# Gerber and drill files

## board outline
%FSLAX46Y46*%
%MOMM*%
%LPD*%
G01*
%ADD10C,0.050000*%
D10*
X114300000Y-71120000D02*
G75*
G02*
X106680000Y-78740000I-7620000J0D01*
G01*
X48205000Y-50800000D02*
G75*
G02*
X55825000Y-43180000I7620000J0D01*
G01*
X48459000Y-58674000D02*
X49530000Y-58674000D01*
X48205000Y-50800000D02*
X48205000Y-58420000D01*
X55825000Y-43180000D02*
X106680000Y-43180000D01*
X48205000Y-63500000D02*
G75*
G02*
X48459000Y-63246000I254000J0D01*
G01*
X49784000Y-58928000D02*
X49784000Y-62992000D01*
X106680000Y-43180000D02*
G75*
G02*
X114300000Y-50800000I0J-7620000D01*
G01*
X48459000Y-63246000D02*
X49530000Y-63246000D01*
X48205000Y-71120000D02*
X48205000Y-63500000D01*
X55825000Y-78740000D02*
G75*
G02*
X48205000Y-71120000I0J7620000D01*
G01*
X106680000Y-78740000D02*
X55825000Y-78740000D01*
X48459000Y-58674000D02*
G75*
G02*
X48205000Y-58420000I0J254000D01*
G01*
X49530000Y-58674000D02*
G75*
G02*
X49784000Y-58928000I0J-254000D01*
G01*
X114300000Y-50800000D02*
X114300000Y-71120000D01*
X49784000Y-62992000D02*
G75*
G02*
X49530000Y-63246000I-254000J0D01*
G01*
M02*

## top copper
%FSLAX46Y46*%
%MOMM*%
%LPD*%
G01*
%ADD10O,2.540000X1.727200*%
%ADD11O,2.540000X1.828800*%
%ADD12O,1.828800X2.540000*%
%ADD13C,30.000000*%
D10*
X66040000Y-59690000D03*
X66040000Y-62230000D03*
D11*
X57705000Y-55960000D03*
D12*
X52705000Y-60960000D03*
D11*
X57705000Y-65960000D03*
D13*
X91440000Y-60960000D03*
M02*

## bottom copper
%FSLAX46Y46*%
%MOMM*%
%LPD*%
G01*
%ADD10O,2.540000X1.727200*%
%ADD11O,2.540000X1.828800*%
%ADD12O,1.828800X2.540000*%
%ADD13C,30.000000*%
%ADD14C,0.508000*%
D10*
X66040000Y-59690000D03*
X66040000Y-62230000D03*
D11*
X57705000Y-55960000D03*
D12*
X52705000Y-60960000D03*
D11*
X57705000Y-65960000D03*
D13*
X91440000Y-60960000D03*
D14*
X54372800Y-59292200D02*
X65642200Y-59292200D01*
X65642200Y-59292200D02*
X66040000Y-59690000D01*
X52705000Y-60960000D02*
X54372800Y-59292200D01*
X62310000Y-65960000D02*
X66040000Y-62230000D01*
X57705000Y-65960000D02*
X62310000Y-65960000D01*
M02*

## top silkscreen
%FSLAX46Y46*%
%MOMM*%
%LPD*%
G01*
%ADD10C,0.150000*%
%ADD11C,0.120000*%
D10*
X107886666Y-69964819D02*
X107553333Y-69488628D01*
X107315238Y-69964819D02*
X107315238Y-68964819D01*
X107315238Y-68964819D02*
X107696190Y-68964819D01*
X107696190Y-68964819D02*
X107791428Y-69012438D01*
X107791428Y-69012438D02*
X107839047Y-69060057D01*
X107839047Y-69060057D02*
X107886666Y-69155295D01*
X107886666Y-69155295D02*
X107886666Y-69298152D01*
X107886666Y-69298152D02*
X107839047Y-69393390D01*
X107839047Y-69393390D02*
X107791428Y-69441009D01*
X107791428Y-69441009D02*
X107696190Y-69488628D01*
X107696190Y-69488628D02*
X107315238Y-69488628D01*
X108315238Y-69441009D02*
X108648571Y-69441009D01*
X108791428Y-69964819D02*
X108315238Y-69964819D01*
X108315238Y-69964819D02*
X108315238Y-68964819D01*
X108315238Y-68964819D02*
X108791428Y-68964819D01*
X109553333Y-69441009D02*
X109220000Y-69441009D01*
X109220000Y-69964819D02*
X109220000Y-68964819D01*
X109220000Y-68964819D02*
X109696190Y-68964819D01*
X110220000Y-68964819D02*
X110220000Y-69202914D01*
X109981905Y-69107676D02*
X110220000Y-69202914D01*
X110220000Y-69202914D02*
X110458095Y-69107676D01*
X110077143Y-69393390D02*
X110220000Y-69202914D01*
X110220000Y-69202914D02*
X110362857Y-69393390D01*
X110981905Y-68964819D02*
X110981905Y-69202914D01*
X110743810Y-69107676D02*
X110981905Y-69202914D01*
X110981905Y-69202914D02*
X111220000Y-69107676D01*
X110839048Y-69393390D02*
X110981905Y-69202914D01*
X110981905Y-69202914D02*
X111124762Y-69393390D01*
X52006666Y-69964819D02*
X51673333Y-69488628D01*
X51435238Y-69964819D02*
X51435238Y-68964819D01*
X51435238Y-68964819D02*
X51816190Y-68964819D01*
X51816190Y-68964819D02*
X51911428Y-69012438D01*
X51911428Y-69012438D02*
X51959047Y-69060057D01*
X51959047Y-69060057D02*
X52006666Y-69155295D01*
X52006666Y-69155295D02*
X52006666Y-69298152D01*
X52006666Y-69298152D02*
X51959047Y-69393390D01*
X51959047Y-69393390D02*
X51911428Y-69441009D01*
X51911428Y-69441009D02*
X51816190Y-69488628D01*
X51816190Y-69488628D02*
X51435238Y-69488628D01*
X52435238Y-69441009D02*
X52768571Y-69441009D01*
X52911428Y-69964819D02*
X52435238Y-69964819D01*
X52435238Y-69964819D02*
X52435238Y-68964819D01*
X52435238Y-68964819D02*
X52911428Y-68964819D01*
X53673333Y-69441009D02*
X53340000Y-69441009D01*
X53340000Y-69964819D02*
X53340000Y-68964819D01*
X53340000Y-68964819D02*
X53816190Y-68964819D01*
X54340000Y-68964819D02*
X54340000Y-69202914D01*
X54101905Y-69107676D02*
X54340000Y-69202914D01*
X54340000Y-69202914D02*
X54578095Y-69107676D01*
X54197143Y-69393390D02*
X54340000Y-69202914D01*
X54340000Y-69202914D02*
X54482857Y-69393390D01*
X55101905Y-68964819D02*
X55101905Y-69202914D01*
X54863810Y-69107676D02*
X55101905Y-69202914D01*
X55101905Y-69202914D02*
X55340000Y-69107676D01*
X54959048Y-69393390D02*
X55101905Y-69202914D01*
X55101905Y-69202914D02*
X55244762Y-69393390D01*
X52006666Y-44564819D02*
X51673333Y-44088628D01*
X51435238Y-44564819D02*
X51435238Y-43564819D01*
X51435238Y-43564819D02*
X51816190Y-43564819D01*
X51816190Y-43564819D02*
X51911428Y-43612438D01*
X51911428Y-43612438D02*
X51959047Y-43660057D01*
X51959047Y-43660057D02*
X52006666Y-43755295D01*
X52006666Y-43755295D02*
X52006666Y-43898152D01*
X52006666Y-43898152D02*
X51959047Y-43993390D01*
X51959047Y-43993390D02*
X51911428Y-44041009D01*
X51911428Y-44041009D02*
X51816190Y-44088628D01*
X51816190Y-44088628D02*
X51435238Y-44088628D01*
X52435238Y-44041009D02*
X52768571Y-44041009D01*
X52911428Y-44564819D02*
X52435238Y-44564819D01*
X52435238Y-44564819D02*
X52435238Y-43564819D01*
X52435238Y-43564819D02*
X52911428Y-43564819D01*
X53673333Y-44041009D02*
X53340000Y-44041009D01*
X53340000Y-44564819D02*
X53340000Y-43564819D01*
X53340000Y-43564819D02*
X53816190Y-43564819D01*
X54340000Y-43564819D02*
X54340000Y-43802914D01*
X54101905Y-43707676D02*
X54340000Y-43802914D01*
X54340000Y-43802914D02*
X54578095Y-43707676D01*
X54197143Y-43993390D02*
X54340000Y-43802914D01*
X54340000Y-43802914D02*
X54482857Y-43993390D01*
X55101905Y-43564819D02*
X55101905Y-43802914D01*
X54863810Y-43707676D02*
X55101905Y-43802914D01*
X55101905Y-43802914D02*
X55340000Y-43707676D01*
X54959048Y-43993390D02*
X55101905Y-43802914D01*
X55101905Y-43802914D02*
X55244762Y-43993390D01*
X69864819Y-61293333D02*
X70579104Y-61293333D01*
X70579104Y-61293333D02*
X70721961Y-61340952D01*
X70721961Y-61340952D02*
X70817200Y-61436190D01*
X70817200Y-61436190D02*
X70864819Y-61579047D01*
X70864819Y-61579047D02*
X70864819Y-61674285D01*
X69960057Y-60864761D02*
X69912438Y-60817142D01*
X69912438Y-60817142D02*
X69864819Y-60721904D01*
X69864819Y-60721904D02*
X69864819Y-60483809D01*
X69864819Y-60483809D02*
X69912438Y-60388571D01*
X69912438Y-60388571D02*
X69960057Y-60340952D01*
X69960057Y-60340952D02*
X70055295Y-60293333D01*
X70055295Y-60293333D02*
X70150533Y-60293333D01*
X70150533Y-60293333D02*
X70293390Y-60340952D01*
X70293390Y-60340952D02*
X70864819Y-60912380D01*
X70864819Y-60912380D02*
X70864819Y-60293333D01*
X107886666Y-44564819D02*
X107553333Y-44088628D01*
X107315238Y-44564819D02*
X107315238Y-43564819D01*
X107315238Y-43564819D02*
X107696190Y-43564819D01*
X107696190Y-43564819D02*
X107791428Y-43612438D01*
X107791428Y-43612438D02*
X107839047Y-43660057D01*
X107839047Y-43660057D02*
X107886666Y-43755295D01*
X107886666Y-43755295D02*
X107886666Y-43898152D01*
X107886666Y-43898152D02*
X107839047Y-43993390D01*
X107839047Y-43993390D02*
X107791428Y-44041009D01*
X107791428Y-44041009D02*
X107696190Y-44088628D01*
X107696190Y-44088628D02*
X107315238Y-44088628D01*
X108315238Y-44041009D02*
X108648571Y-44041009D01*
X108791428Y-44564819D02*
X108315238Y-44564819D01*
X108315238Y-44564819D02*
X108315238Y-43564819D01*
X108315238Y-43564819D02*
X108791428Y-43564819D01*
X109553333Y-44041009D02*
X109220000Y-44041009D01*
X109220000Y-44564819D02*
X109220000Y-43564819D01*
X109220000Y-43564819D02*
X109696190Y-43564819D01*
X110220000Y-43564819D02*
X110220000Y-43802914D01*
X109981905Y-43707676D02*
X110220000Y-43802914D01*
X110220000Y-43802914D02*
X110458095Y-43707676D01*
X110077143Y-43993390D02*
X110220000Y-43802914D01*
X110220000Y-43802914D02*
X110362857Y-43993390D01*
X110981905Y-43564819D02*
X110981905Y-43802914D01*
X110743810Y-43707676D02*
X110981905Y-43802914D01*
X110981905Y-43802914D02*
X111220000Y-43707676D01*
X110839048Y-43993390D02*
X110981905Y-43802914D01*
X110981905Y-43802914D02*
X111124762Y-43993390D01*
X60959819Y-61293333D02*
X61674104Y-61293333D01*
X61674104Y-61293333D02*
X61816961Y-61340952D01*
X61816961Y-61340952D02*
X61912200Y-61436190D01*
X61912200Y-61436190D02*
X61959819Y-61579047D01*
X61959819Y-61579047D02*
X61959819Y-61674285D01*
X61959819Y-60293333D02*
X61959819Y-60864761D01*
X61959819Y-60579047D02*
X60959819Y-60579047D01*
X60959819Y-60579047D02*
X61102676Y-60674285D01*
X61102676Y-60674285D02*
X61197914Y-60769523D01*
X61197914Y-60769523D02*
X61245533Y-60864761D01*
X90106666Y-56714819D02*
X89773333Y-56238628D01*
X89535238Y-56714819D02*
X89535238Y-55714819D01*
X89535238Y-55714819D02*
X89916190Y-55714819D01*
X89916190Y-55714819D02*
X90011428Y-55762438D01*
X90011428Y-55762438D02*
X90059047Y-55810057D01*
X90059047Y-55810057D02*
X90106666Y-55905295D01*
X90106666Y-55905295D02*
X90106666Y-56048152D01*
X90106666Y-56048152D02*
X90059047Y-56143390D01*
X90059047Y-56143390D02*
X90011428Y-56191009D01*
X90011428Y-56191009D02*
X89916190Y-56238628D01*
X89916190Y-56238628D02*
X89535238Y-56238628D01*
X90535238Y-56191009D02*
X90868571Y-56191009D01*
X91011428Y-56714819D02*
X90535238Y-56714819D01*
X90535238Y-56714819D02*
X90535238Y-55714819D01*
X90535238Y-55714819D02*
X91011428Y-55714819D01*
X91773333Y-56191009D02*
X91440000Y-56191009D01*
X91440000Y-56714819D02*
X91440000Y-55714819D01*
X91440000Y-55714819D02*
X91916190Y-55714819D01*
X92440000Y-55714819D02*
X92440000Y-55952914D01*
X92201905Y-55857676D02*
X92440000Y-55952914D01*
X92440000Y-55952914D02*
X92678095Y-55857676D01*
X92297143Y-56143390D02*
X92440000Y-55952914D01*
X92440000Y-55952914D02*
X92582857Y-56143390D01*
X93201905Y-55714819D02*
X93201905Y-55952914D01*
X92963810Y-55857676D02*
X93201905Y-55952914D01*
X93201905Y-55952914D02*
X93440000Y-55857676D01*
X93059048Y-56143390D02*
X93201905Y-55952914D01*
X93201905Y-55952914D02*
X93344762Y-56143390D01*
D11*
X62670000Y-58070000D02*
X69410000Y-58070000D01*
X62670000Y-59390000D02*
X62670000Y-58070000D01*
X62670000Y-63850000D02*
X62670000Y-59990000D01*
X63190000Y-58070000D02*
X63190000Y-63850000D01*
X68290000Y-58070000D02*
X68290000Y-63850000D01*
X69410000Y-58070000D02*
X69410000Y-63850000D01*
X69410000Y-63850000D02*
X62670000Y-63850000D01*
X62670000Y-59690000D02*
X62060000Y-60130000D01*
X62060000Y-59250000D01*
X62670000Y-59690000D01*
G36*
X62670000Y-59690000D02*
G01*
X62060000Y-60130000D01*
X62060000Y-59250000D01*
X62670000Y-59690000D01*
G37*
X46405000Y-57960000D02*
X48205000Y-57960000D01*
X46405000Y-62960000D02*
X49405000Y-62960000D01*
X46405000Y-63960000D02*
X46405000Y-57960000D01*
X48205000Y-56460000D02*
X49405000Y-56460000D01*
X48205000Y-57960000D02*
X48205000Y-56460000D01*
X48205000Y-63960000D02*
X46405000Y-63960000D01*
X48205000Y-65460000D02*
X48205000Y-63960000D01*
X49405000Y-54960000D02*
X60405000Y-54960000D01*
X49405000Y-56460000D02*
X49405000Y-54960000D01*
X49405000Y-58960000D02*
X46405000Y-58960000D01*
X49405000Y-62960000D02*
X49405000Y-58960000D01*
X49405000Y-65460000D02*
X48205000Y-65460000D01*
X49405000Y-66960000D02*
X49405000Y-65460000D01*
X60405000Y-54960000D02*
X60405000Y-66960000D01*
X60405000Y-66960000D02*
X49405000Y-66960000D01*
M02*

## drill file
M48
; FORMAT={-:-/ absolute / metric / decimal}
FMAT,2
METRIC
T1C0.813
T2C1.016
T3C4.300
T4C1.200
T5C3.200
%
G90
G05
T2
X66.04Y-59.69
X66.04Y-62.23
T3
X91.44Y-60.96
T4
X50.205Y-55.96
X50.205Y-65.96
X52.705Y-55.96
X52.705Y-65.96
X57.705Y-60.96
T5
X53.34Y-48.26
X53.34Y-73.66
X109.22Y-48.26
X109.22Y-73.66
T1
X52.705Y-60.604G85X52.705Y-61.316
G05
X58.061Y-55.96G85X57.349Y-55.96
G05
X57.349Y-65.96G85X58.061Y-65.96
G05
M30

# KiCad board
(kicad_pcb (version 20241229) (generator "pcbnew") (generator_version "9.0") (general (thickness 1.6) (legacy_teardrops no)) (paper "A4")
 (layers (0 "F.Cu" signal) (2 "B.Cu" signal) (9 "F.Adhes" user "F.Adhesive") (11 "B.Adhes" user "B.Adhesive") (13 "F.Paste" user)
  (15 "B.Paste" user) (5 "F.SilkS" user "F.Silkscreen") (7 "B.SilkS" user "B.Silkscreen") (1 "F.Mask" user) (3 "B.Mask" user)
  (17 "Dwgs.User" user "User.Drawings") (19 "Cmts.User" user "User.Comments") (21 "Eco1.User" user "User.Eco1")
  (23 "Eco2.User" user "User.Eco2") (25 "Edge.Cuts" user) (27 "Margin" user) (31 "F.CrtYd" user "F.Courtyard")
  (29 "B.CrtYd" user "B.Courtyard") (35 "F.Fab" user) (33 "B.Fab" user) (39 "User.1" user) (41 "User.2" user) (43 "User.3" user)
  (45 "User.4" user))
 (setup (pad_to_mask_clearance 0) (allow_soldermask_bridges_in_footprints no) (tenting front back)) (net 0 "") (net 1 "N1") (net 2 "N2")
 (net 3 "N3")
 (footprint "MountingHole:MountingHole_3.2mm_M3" (layer "F.Cu") (at 109.22 73.66)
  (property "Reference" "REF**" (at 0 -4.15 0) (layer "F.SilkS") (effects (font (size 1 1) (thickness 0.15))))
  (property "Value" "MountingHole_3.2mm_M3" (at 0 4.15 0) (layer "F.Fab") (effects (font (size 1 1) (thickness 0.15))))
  (pad "" np_thru_hole circle (at 0 0) (size 3.2 3.2) (drill 3.2) (layers "*.Cu" "*.Mask")))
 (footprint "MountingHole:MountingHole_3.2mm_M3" (layer "F.Cu") (at 53.34 73.66)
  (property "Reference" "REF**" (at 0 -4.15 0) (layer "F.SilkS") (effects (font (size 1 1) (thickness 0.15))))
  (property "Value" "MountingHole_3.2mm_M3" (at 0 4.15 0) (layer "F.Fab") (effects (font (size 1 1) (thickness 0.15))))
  (pad "" np_thru_hole circle (at 0 0) (size 3.2 3.2) (drill 3.2) (layers "*.Cu" "*.Mask")))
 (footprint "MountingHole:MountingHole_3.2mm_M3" (layer "F.Cu") (at 53.34 48.26)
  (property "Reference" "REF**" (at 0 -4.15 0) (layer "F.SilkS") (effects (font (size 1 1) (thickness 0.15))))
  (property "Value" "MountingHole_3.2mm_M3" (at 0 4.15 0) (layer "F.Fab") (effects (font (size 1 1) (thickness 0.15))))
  (pad "" np_thru_hole circle (at 0 0) (size 3.2 3.2) (drill 3.2) (layers "*.Cu" "*.Mask")))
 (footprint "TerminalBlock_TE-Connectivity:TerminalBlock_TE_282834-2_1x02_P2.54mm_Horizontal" (layer "F.Cu") (at 66.04 59.69 -90)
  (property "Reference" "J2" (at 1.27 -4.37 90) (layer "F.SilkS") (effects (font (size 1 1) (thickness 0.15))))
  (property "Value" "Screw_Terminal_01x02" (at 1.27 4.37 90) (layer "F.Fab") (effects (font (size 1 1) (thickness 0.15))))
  (fp_line (start -1.62 3.37) (end -1.62 -3.37) (stroke (width 0.12) (type solid)) (layer "F.SilkS"))
  (fp_line (start -0.3 3.37) (end -1.62 3.37) (stroke (width 0.12) (type solid)) (layer "F.SilkS"))
  (fp_line (start 4.16 3.37) (end 0.3 3.37) (stroke (width 0.12) (type solid)) (layer "F.SilkS"))
  (fp_line (start -1.62 2.85) (end 4.16 2.85) (stroke (width 0.12) (type solid)) (layer "F.SilkS"))
  (fp_line (start -1.62 -2.25) (end 4.16 -2.25) (stroke (width 0.12) (type solid)) (layer "F.SilkS"))
  (fp_line (start -1.62 -3.37) (end 4.16 -3.37) (stroke (width 0.12) (type solid)) (layer "F.SilkS"))
  (fp_line (start 4.16 -3.37) (end 4.16 3.37) (stroke (width 0.12) (type solid)) (layer "F.SilkS"))
  (fp_poly (pts (xy 0 3.37) (xy 0.44 3.98) (xy -0.44 3.98)) (stroke (width 0.12) (type solid)) (fill yes) (layer "F.SilkS"))
  (pad "1" thru_hole oval (at 0 0 270) (size 1.7272 2.54) (drill 1.016) (layers "*.Cu" "*.Mask") (remove_unused_layers no) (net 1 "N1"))
  (pad "2" thru_hole oval (at 2.54 0 270) (size 1.7272 2.54) (drill 1.016) (layers "*.Cu" "*.Mask") (remove_unused_layers no) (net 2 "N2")))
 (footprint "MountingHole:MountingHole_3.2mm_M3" (layer "F.Cu") (at 109.22 48.26)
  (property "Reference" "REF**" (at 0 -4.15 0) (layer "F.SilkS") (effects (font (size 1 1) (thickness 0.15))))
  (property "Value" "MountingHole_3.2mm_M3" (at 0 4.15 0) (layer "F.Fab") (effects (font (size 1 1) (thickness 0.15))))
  (pad "" np_thru_hole circle (at 0 0) (size 3.2 3.2) (drill 3.2) (layers "*.Cu" "*.Mask")))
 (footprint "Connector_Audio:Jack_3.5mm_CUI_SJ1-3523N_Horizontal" (layer "F.Cu") (at 52.705 60.96 -90)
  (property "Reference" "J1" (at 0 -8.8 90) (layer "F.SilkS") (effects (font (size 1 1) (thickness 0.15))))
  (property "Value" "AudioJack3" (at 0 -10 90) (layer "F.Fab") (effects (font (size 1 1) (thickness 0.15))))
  (fp_line (start -3 6.3) (end -3 4.5) (stroke (width 0.12) (type solid)) (layer "F.SilkS"))
  (fp_line (start 2 6.3) (end 2 3.3) (stroke (width 0.12) (type solid)) (layer "F.SilkS"))
  (fp_line (start 3 6.3) (end -3 6.3) (stroke (width 0.12) (type solid)) (layer "F.SilkS"))
  (fp_line (start -4.5 4.5) (end -4.5 3.3) (stroke (width 0.12) (type solid)) (layer "F.SilkS"))
  (fp_line (start -3 4.5) (end -4.5 4.5) (stroke (width 0.12) (type solid)) (layer "F.SilkS"))
  (fp_line (start 3 4.5) (end 3 6.3) (stroke (width 0.12) (type solid)) (layer "F.SilkS"))
  (fp_line (start 4.5 4.5) (end 3 4.5) (stroke (width 0.12) (type solid)) (layer "F.SilkS"))
  (fp_line (start -6 3.3) (end -6 -7.7) (stroke (width 0.12) (type solid)) (layer "F.SilkS"))
  (fp_line (start -4.5 3.3) (end -6 3.3) (stroke (width 0.12) (type solid)) (layer "F.SilkS"))
  (fp_line (start -2 3.3) (end -2 6.3) (stroke (width 0.12) (type solid)) (layer "F.SilkS"))
  (fp_line (start 2 3.3) (end -2 3.3) (stroke (width 0.12) (type solid)) (layer "F.SilkS"))
  (fp_line (start 4.5 3.3) (end 4.5 4.5) (stroke (width 0.12) (type solid)) (layer "F.SilkS"))
  (fp_line (start 6 3.3) (end 4.5 3.3) (stroke (width 0.12) (type solid)) (layer "F.SilkS"))
  (fp_line (start -6 -7.7) (end 6 -7.7) (stroke (width 0.12) (type solid)) (layer "F.SilkS"))
  (fp_line (start 6 -7.7) (end 6 3.3) (stroke (width 0.12) (type solid)) (layer "F.SilkS"))
  (pad "" np_thru_hole circle (at -5 0 270) (size 1.2 1.2) (drill 1.2) (layers "*.Cu" "*.Mask"))
  (pad "" np_thru_hole circle (at -5 2.5 270) (size 1.2 1.2) (drill 1.2) (layers "*.Cu" "*.Mask"))
  (pad "" np_thru_hole circle (at 0 -5 270) (size 1.2 1.2) (drill 1.2) (layers "*.Cu" "*.Mask"))
  (pad "" np_thru_hole circle (at 5 0 270) (size 1.2 1.2) (drill 1.2) (layers "*.Cu" "*.Mask"))
  (pad "" np_thru_hole circle (at 5 2.5 270) (size 1.2 1.2) (drill 1.2) (layers "*.Cu" "*.Mask"))
  (pad "R" thru_hole oval (at -5 -5 270) (size 1.8288 2.54) (drill oval 0.8128 1.524) (layers "*.Cu" "*.Mask") (remove_unused_layers no)
   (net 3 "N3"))
  (pad "S" thru_hole oval (at 0 0 270) (size 2.54 1.8288) (drill oval 1.524 0.8128) (layers "*.Cu" "*.Mask") (remove_unused_layers no)
   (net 1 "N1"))
  (pad "T" thru_hole oval (at 5 -5 90) (size 1.8288 2.54) (drill oval 0.8128 1.524) (layers "*.Cu" "*.Mask") (remove_unused_layers no)
   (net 2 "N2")))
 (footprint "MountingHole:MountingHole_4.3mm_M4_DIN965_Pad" (layer "F.Cu") (at 91.44 60.96)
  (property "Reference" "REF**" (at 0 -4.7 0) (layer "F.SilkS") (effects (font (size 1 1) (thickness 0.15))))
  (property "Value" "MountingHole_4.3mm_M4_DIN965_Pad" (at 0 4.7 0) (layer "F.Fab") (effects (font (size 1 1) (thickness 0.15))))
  (pad "1" thru_hole circle (at 0 0) (size 30 30) (drill 4.3) (layers "*.Cu" "*.Mask") (remove_unused_layers no) (zone_connect 2)))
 (gr_arc (start 114.3 71.12) (mid 112.068154 76.508154) (end 106.68 78.74) (stroke (width 0.05) (type default)) (layer "Edge.Cuts"))
 (gr_arc (start 48.205 50.8) (mid 50.436846 45.411846) (end 55.825 43.18) (stroke (width 0.05) (type default)) (layer "Edge.Cuts"))
 (gr_line (start 48.459 58.674) (end 49.53 58.674) (stroke (width 0.05) (type default)) (layer "Edge.Cuts"))
 (gr_line (start 48.205 50.8) (end 48.205 58.42) (stroke (width 0.05) (type default)) (layer "Edge.Cuts"))
 (gr_line (start 55.825 43.18) (end 106.68 43.18) (stroke (width 0.05) (type default)) (layer "Edge.Cuts"))
 (gr_arc (start 48.205 63.5) (mid 48.279395 63.320395) (end 48.459 63.246) (stroke (width 0.05) (type default)) (layer "Edge.Cuts"))
 (gr_line (start 49.784 58.928) (end 49.784 62.992) (stroke (width 0.05) (type default)) (layer "Edge.Cuts"))
 (gr_arc (start 106.68 43.18) (mid 112.068154 45.411846) (end 114.3 50.8) (stroke (width 0.05) (type default)) (layer "Edge.Cuts"))
 (gr_line (start 48.459 63.246) (end 49.53 63.246) (stroke (width 0.05) (type default)) (layer "Edge.Cuts"))
 (gr_line (start 48.205 71.12) (end 48.205 63.5) (stroke (width 0.05) (type default)) (layer "Edge.Cuts"))
 (gr_arc (start 55.825 78.74) (mid 50.436846 76.508154) (end 48.205 71.12) (stroke (width 0.05) (type default)) (layer "Edge.Cuts"))
 (gr_line (start 106.68 78.74) (end 55.825 78.74) (stroke (width 0.05) (type default)) (layer "Edge.Cuts"))
 (gr_arc (start 48.459 58.674) (mid 48.279395 58.599605) (end 48.205 58.42) (stroke (width 0.05) (type default)) (layer "Edge.Cuts"))
 (gr_arc (start 49.53 58.674) (mid 49.709605 58.748395) (end 49.784 58.928) (stroke (width 0.05) (type default)) (layer "Edge.Cuts"))
 (gr_line (start 114.3 50.8) (end 114.3 71.12) (stroke (width 0.05) (type default)) (layer "Edge.Cuts"))
 (gr_arc (start 49.784 62.992) (mid 49.709605 63.171605) (end 49.53 63.246) (stroke (width 0.05) (type default)) (layer "Edge.Cuts"))
 (segment (start 54.3728 59.2922) (end 65.6422 59.2922) (width 0.508) (layer "B.Cu") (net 1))
 (segment (start 65.6422 59.2922) (end 66.04 59.69) (width 0.508) (layer "B.Cu") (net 1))
 (segment (start 52.705 60.96) (end 54.3728 59.2922) (width 0.508) (layer "B.Cu") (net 1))
 (segment (start 62.31 65.96) (end 66.04 62.23) (width 0.508) (layer "B.Cu") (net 2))
 (segment (start 57.705 65.96) (end 62.31 65.96) (width 0.508) (layer "B.Cu") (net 2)))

